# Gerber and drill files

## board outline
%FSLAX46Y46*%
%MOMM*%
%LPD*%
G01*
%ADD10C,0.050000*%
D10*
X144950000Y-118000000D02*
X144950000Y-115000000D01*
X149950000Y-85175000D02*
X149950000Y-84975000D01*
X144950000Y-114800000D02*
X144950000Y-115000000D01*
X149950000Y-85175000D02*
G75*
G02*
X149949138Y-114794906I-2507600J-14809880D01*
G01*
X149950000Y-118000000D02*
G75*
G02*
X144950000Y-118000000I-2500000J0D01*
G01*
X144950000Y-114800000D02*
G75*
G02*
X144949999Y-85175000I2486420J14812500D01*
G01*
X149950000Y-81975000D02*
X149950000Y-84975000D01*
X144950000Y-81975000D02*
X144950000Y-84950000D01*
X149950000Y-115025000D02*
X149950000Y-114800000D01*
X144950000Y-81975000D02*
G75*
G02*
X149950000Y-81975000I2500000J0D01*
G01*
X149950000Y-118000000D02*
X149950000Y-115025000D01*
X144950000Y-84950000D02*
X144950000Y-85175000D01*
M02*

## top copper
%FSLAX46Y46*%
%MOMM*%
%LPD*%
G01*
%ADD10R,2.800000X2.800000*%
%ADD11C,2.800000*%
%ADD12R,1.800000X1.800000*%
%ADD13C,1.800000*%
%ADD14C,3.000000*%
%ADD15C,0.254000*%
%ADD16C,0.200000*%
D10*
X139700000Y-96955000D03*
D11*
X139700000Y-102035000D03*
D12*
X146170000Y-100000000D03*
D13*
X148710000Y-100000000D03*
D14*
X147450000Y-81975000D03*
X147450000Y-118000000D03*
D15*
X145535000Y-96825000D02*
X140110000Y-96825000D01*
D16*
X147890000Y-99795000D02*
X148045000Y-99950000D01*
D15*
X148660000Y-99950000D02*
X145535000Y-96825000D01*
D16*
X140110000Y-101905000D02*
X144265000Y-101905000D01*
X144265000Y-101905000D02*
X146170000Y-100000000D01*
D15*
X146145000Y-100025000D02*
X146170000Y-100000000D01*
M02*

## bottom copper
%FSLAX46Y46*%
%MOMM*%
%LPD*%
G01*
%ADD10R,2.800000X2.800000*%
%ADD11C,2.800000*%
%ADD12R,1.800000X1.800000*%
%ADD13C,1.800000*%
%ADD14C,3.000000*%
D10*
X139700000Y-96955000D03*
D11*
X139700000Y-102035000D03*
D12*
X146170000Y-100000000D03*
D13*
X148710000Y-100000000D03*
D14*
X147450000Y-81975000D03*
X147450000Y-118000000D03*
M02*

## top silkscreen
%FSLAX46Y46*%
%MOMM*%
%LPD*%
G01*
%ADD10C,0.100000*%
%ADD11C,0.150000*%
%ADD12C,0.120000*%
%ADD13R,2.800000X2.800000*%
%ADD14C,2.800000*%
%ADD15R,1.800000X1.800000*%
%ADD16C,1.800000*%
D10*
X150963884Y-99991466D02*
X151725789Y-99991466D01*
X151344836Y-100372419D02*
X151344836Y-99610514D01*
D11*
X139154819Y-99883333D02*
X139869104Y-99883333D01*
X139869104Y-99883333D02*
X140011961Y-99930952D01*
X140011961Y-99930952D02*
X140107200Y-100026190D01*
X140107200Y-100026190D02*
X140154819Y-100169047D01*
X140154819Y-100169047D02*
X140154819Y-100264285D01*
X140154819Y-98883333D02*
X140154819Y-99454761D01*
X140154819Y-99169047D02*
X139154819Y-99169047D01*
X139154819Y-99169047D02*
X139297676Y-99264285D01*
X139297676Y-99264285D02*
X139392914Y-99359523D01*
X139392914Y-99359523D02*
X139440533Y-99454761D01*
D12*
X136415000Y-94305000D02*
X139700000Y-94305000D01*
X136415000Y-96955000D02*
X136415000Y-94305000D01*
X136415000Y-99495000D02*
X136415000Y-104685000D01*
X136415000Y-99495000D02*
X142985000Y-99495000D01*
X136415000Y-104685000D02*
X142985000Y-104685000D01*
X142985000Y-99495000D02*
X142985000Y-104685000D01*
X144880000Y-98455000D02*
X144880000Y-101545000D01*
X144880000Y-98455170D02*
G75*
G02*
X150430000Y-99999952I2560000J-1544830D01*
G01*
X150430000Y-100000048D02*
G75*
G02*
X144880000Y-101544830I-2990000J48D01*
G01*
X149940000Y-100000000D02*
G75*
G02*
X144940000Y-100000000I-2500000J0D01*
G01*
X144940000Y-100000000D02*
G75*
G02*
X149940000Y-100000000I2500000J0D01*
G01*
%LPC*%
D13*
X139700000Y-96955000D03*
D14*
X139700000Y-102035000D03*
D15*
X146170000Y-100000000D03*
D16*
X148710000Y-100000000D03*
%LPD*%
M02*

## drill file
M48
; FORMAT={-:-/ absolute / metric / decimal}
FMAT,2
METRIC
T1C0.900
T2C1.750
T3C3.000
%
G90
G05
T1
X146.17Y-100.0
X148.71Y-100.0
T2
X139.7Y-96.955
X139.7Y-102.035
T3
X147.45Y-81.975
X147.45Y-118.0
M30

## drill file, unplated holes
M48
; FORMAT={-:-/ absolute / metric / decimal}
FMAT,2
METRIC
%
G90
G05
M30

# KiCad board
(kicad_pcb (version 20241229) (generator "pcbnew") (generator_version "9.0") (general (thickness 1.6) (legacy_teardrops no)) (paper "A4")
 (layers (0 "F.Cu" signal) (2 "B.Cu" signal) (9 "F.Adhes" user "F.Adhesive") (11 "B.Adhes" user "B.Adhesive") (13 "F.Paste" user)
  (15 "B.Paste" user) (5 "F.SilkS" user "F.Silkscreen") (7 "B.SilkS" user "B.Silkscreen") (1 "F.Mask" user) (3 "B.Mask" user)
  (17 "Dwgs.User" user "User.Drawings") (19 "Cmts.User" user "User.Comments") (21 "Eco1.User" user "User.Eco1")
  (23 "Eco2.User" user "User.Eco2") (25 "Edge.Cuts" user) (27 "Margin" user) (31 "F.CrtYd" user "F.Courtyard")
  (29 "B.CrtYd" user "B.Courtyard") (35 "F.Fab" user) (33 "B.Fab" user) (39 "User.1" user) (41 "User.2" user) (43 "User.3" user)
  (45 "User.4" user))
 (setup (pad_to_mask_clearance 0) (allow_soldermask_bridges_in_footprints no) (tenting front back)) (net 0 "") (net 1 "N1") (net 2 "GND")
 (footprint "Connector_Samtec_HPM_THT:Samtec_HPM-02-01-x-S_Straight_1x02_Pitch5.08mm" (layer "F.Cu") (at 139.7 96.955)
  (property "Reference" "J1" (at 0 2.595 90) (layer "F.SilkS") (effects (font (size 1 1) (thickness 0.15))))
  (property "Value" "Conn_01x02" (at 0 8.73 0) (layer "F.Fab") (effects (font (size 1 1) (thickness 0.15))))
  (fp_line (start -3.285 -2.65) (end 0 -2.65) (stroke (width 0.12) (type solid)) (layer "F.SilkS"))
  (fp_line (start -3.285 0) (end -3.285 -2.65) (stroke (width 0.12) (type solid)) (layer "F.SilkS"))
  (fp_line (start -3.285 2.54) (end -3.285 7.73) (stroke (width 0.12) (type solid)) (layer "F.SilkS"))
  (fp_line (start -3.285 2.54) (end 3.285 2.54) (stroke (width 0.12) (type solid)) (layer "F.SilkS"))
  (fp_line (start -3.285 7.73) (end 3.285 7.73) (stroke (width 0.12) (type solid)) (layer "F.SilkS"))
  (fp_line (start 3.285 2.54) (end 3.285 7.73) (stroke (width 0.12) (type solid)) (layer "F.SilkS"))
  (pad "1" thru_hole rect (at 0 0) (size 2.8 2.8) (drill 1.75) (layers "*.Cu" "*.Mask") (remove_unused_layers no) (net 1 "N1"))
  (pad "2" thru_hole circle (at 0 5.08) (size 2.8 2.8) (drill 1.75) (layers "*.Cu" "*.Mask") (remove_unused_layers no) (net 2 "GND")))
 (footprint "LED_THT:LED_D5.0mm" (layer "F.Cu") (at 146.17 100)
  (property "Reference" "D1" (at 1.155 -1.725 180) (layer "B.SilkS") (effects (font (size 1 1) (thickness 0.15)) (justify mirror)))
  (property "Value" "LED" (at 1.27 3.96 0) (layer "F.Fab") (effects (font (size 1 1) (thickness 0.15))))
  (fp_line (start -1.29 -1.545) (end -1.29 1.545) (stroke (width 0.12) (type solid)) (layer "F.SilkS"))
  (fp_arc (start -1.29 -1.54483) (mid 2.071756 -2.880501) (end 4.26 -0.000048) (stroke (width 0.12) (type solid)) (layer "F.SilkS"))
  (fp_arc (start 4.26 0.000048) (mid 2.071756 2.880501) (end -1.29 1.54483) (stroke (width 0.12) (type solid)) (layer "F.SilkS"))
  (fp_circle (center 1.27 0) (end 3.77 0) (stroke (width 0.12) (type solid)) (fill no) (layer "F.SilkS"))
  (pad "1" thru_hole rect (at 0 0) (size 1.8 1.8) (drill 0.9) (layers "*.Cu" "*.Mask") (remove_unused_layers no) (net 2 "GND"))
  (pad "2" thru_hole circle (at 2.54 0) (size 1.8 1.8) (drill 0.9) (layers "*.Cu" "*.Mask") (remove_unused_layers no) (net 1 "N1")))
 (gr_line (start 144.95 118) (end 144.95 115) (stroke (width 0.05) (type default)) (layer "Edge.Cuts"))
 (gr_line (start 149.95 85.175) (end 149.95 84.975) (stroke (width 0.05) (type default)) (layer "Edge.Cuts"))
 (gr_line (start 144.95 114.8) (end 144.95 115) (stroke (width 0.05) (type default)) (layer "Edge.Cuts"))
 (gr_arc (start 149.95 85.175) (mid 162.463074 99.985336) (end 149.949138 114.794908) (stroke (width 0.05) (type default))
  (layer "Edge.Cuts"))
 (gr_arc (start 149.95 118) (mid 147.45 120.5) (end 144.95 118) (stroke (width 0.05) (type default)) (layer "Edge.Cuts"))
 (gr_arc (start 144.95 114.8) (mid 132.416686 99.9875) (end 144.949999 85.175) (stroke (width 0.05) (type default)) (layer "Edge.Cuts"))
 (gr_line (start 149.95 81.975) (end 149.95 84.975) (stroke (width 0.05) (type default)) (layer "Edge.Cuts"))
 (gr_line (start 144.95 81.975) (end 144.95 84.95) (stroke (width 0.05) (type default)) (layer "Edge.Cuts"))
 (gr_line (start 149.95 115.025) (end 149.95 114.8) (stroke (width 0.05) (type default)) (layer "Edge.Cuts"))
 (gr_arc (start 144.95 81.975) (mid 147.45 79.475) (end 149.95 81.975) (stroke (width 0.05) (type default)) (layer "Edge.Cuts"))
 (gr_line (start 149.95 118) (end 149.95 115.025) (stroke (width 0.05) (type default)) (layer "Edge.Cuts"))
 (gr_line (start 144.95 84.95) (end 144.95 85.175) (stroke (width 0.05) (type default)) (layer "Edge.Cuts"))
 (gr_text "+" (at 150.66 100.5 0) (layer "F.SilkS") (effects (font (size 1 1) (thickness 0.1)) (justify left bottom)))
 (via (at 147.45 81.975) (size 3) (drill 3) (layers "F.Cu" "B.Cu") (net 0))
 (via (at 147.45 118) (size 3) (drill 3) (layers "F.Cu" "B.Cu") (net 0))
 (segment (start 145.535 96.825) (end 140.11 96.825) (width 0.254) (layer "F.Cu") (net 1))
 (segment (start 147.89 99.795) (end 148.045 99.95) (width 0.2) (layer "F.Cu") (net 1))
 (segment (start 148.66 99.95) (end 145.535 96.825) (width 0.254) (layer "F.Cu") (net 1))
 (segment (start 140.11 101.905) (end 144.265 101.905) (width 0.2) (layer "F.Cu") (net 2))
 (segment (start 144.265 101.905) (end 146.17 100) (width 0.2) (layer "F.Cu") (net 2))
 (segment (start 146.145 100.025) (end 146.17 100) (width 0.254) (layer "F.Cu") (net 2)))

